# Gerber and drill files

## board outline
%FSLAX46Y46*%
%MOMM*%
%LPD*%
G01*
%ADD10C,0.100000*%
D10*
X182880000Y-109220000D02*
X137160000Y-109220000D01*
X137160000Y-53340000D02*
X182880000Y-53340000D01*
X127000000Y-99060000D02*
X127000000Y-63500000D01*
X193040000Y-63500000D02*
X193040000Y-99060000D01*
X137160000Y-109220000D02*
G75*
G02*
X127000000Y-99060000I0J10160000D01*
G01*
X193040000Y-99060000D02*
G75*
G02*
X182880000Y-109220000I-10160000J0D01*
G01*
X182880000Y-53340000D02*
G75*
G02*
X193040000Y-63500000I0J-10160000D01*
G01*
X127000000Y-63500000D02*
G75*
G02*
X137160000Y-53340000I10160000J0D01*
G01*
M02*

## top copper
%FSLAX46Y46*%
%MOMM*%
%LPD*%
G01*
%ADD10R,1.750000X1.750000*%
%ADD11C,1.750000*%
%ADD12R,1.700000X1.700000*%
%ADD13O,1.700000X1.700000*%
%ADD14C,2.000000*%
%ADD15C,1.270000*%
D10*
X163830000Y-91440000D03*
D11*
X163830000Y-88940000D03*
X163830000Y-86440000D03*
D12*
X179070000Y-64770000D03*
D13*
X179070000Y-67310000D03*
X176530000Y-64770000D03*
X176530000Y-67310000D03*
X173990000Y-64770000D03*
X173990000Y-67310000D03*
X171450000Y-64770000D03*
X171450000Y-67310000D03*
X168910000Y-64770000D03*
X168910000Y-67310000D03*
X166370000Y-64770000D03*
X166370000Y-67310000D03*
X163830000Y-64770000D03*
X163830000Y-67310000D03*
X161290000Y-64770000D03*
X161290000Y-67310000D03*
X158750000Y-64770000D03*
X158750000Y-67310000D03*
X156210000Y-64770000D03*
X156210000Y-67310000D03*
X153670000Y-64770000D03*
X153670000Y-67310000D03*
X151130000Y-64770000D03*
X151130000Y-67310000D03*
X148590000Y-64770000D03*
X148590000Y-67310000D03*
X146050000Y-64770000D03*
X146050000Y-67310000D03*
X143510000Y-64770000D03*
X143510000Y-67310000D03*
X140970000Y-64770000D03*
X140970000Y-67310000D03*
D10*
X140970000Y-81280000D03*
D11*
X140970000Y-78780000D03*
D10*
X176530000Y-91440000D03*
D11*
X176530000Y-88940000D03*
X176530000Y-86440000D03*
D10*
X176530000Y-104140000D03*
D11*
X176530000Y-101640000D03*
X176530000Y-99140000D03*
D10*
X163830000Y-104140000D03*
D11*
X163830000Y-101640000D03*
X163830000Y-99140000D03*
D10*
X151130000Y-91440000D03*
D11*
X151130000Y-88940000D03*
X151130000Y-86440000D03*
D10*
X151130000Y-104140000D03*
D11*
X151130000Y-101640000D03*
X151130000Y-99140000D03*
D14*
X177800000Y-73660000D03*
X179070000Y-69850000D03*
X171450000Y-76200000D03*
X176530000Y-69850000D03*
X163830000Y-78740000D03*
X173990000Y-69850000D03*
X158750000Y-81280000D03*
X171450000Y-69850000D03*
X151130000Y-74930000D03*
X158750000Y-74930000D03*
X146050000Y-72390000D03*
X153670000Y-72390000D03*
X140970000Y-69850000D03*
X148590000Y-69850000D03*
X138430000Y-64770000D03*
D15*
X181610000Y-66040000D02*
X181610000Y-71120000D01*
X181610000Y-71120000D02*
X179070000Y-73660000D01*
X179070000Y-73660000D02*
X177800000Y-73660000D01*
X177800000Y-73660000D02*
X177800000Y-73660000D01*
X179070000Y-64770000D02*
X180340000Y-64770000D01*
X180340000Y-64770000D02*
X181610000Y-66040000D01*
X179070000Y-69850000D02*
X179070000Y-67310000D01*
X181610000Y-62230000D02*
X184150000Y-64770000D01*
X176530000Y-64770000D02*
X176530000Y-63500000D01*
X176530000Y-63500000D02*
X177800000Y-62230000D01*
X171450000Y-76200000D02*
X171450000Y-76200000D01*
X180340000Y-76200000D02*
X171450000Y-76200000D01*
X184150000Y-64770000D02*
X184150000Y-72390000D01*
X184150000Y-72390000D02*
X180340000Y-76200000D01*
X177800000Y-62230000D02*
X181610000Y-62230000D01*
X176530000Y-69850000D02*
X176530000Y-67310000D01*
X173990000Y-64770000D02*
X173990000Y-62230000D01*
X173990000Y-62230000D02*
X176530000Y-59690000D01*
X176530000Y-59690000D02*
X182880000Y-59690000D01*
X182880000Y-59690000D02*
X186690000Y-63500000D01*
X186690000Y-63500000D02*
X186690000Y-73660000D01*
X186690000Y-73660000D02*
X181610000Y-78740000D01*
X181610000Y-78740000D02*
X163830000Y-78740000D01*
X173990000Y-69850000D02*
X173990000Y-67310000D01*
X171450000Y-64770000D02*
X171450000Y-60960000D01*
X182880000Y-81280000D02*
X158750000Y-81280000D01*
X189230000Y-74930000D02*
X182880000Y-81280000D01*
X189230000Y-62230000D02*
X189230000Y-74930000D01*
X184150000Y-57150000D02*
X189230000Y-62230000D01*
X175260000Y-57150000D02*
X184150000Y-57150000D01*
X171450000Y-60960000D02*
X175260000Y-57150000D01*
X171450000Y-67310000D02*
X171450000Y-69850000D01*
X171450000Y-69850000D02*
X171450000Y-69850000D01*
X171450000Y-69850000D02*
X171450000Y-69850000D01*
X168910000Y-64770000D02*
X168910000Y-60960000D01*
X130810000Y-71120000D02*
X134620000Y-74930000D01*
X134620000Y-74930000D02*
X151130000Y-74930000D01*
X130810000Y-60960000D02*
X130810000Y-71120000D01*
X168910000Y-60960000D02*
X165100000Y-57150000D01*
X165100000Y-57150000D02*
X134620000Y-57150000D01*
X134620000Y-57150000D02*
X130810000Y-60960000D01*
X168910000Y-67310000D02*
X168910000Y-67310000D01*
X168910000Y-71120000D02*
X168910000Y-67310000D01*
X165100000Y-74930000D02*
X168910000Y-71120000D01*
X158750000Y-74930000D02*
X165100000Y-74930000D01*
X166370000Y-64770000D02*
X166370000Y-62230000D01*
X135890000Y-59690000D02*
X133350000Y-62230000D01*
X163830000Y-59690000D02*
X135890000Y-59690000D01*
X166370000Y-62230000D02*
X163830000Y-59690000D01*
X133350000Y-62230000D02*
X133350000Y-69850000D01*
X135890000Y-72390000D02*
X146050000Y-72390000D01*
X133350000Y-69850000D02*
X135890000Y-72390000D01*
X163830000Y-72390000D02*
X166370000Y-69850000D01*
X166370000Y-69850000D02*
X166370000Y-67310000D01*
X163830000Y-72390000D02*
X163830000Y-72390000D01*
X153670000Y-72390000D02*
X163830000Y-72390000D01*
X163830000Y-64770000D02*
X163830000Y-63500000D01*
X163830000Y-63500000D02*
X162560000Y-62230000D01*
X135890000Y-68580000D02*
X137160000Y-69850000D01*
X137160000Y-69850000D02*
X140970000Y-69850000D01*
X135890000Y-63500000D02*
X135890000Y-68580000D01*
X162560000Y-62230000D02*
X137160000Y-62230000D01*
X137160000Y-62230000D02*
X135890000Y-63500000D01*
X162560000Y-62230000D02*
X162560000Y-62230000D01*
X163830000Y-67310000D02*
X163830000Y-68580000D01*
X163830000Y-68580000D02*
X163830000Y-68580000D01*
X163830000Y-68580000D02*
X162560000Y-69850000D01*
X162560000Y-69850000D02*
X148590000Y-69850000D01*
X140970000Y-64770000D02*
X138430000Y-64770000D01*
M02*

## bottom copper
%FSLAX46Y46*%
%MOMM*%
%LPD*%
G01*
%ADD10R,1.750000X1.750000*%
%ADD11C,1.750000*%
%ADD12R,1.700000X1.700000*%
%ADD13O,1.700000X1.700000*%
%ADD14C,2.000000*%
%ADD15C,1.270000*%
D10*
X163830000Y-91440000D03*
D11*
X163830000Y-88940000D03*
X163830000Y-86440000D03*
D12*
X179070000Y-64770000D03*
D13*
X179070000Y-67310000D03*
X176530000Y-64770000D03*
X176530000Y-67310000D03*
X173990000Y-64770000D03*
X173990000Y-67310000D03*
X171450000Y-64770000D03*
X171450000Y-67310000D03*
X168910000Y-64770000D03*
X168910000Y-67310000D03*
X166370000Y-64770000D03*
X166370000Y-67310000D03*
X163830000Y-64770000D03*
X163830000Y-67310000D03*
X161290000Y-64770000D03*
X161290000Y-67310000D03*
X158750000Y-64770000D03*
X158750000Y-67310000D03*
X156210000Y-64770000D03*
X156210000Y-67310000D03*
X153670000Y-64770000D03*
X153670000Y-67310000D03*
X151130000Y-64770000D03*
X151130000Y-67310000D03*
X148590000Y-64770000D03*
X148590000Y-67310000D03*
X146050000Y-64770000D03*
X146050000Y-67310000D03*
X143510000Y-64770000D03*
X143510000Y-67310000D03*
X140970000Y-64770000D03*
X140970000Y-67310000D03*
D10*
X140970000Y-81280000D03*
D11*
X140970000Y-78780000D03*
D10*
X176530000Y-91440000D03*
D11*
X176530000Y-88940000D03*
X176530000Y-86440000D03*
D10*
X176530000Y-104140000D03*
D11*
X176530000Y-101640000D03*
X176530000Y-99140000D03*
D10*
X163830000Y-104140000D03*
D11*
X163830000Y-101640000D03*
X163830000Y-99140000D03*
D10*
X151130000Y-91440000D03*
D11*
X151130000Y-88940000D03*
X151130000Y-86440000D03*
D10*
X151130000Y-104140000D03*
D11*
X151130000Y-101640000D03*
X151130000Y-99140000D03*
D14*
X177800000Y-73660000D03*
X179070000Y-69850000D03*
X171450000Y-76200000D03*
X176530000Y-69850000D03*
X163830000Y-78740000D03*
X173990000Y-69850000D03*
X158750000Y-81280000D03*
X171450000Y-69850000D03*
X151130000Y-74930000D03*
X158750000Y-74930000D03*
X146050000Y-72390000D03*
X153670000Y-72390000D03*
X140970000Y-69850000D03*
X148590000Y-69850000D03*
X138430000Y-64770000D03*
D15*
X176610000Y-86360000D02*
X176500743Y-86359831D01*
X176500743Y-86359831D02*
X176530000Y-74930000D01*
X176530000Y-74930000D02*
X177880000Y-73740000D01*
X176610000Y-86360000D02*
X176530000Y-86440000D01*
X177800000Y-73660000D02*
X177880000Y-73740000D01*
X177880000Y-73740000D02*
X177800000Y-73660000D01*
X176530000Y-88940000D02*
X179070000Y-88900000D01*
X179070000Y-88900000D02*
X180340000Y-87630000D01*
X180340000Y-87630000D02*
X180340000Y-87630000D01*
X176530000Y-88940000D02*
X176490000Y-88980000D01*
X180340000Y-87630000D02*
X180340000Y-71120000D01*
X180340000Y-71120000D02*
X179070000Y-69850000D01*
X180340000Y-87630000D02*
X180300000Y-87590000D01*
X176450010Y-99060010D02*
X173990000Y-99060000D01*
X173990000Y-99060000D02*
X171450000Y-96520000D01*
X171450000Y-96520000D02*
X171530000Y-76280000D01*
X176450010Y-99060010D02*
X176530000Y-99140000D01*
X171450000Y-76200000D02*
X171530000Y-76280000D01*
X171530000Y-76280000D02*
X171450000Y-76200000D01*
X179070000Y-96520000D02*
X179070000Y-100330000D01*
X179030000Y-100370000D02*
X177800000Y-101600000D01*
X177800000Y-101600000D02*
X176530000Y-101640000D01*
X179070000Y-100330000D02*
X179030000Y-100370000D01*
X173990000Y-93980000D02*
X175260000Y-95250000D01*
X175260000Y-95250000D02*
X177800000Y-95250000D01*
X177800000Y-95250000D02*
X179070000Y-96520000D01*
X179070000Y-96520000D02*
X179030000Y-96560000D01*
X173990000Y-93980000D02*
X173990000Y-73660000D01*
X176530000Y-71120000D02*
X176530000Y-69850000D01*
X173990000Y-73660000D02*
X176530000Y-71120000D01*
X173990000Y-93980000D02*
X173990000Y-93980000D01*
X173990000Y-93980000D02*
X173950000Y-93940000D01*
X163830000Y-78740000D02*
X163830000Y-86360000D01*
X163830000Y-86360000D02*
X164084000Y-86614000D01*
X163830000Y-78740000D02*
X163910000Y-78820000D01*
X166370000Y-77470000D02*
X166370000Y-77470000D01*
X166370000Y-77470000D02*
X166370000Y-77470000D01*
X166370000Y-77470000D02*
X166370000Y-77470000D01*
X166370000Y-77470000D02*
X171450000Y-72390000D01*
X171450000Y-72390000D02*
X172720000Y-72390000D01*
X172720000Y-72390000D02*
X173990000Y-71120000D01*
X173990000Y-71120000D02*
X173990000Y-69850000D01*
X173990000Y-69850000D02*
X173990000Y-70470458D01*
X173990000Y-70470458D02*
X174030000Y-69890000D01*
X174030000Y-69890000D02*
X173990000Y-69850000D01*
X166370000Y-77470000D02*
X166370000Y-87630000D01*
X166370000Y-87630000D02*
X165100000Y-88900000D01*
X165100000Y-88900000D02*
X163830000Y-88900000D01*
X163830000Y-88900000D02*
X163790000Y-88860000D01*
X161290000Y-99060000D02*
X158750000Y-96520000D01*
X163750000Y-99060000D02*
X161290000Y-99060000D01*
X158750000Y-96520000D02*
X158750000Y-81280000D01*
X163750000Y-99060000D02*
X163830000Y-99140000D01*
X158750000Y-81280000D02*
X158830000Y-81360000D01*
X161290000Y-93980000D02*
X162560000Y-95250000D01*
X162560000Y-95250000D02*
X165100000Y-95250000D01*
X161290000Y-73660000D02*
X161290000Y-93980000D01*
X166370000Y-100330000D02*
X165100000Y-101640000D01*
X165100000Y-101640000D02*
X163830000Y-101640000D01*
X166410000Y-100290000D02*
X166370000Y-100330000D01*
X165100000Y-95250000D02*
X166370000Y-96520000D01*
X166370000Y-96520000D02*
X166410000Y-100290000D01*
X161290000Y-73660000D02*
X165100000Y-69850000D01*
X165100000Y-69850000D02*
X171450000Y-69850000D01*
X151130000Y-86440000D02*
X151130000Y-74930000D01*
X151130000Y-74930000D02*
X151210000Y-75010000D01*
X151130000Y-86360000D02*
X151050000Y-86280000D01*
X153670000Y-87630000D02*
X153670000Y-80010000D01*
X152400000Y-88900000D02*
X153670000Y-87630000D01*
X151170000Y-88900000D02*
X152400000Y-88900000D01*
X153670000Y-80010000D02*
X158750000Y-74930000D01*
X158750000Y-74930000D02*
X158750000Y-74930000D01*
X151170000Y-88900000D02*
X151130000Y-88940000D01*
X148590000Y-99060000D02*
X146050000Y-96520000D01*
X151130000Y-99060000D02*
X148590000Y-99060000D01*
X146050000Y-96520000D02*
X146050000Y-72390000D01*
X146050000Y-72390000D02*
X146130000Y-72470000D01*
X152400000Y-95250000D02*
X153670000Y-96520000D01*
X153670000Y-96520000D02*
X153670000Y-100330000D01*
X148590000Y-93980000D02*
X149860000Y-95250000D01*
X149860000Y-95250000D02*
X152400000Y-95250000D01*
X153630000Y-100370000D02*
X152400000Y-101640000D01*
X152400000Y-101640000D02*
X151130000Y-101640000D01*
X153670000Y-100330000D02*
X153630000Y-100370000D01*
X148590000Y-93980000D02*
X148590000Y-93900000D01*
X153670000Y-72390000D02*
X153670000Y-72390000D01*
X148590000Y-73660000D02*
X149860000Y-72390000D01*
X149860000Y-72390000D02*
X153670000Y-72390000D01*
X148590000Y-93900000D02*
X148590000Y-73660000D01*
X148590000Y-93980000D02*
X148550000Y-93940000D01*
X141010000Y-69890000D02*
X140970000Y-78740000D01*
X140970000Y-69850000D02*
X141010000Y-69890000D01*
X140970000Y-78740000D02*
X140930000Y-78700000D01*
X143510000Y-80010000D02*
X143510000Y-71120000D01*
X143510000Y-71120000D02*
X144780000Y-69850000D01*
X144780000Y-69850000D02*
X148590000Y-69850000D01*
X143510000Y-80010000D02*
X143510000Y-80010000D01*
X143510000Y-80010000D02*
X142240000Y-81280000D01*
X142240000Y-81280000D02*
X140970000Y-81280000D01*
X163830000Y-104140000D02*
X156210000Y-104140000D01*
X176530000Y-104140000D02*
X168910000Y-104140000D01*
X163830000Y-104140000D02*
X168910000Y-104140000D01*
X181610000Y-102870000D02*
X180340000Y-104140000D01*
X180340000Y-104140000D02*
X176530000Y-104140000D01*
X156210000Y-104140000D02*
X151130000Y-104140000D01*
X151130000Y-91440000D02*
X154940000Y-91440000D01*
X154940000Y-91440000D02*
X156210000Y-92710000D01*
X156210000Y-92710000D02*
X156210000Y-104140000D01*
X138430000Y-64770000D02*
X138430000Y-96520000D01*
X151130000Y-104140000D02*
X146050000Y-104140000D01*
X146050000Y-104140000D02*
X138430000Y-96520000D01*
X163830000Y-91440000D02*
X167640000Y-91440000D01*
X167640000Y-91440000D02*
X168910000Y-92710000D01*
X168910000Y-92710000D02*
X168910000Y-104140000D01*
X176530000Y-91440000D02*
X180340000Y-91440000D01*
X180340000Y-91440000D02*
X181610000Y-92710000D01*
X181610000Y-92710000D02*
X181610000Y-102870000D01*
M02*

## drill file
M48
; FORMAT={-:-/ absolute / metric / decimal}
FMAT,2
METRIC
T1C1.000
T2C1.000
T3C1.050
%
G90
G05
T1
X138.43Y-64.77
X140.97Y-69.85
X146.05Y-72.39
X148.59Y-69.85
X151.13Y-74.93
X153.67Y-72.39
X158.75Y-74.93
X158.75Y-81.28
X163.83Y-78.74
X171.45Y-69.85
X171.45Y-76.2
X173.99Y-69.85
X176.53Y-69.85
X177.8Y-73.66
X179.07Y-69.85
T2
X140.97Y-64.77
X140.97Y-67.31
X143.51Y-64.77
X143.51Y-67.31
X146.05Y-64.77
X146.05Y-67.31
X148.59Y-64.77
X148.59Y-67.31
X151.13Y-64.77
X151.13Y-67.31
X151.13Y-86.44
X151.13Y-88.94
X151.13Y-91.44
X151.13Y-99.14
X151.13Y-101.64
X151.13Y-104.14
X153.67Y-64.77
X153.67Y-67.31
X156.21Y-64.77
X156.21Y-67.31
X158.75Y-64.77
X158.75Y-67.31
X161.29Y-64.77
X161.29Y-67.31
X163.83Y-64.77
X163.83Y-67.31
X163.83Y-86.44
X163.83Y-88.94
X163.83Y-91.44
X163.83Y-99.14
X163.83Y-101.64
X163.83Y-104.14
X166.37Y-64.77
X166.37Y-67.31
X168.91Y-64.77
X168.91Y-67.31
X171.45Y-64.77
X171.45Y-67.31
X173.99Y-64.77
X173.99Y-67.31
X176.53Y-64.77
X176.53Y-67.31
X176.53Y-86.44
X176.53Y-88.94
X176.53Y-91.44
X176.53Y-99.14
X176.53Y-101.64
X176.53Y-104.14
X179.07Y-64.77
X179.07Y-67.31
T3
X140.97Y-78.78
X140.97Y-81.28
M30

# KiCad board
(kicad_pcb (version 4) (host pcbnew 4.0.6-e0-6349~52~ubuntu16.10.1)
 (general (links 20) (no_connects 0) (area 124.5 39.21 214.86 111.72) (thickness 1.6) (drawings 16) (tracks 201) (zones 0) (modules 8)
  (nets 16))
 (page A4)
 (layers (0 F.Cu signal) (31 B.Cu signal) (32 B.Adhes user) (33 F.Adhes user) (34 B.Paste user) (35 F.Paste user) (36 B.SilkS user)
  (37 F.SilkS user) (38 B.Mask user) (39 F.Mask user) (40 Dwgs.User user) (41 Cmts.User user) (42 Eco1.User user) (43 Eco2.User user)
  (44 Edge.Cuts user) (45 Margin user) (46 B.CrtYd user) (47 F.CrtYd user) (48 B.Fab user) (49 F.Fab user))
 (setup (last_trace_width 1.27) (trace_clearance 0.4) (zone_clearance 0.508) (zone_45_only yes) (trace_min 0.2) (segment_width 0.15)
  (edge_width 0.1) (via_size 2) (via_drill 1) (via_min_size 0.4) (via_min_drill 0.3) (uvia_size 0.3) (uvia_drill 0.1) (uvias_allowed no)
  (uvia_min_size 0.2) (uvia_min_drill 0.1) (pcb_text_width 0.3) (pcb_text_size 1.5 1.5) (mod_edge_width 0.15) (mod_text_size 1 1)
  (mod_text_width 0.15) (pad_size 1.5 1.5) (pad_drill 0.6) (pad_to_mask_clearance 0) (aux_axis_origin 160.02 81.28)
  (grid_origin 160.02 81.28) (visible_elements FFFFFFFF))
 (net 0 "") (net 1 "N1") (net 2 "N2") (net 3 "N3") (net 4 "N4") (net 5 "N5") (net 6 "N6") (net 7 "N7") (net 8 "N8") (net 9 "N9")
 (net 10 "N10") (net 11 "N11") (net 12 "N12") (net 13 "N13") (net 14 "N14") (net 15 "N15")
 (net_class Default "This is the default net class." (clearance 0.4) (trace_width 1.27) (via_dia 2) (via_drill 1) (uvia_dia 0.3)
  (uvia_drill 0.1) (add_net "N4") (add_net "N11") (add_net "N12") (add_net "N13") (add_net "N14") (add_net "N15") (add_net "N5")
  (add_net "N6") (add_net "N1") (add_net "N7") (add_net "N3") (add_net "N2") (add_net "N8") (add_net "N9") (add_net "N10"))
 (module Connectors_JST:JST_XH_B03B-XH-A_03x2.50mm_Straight (layer F.Cu) (at 163.83 91.44 90)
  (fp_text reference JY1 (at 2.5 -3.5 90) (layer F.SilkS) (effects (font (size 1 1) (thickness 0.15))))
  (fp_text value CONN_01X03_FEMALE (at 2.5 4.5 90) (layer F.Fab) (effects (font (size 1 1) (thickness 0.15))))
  (pad 1 thru_hole rect (at 0 0 90) (size 1.75 1.75) (drill 1) (layers *.Cu *.Mask) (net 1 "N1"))
  (pad 2 thru_hole circle (at 2.5 0 90) (size 1.75 1.75) (drill 1) (layers *.Cu *.Mask) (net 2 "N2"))
  (pad 3 thru_hole circle (at 5 0 90) (size 1.75 1.75) (drill 1) (layers *.Cu *.Mask) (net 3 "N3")))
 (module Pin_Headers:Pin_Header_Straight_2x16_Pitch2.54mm (layer F.Cu) (at 179.07 64.77 270)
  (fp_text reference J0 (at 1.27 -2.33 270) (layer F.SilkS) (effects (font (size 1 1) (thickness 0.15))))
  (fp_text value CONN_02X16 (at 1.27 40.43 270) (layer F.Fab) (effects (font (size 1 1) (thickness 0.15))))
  (pad 1 thru_hole rect (at 0 0 270) (size 1.7 1.7) (drill 1) (layers *.Cu *.Mask) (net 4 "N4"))
  (pad 2 thru_hole oval (at 2.54 0 270) (size 1.7 1.7) (drill 1) (layers *.Cu *.Mask) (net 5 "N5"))
  (pad 3 thru_hole oval (at 0 2.54 270) (size 1.7 1.7) (drill 1) (layers *.Cu *.Mask) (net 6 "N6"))
  (pad 4 thru_hole oval (at 2.54 2.54 270) (size 1.7 1.7) (drill 1) (layers *.Cu *.Mask) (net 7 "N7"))
  (pad 5 thru_hole oval (at 0 5.08 270) (size 1.7 1.7) (drill 1) (layers *.Cu *.Mask) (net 3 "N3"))
  (pad 6 thru_hole oval (at 2.54 5.08 270) (size 1.7 1.7) (drill 1) (layers *.Cu *.Mask) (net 2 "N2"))
  (pad 7 thru_hole oval (at 0 7.62 270) (size 1.7 1.7) (drill 1) (layers *.Cu *.Mask) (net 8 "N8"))
  (pad 8 thru_hole oval (at 2.54 7.62 270) (size 1.7 1.7) (drill 1) (layers *.Cu *.Mask) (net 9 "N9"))
  (pad 9 thru_hole oval (at 0 10.16 270) (size 1.7 1.7) (drill 1) (layers *.Cu *.Mask) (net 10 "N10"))
  (pad 10 thru_hole oval (at 2.54 10.16 270) (size 1.7 1.7) (drill 1) (layers *.Cu *.Mask) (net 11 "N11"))
  (pad 11 thru_hole oval (at 0 12.7 270) (size 1.7 1.7) (drill 1) (layers *.Cu *.Mask) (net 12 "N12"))
  (pad 12 thru_hole oval (at 2.54 12.7 270) (size 1.7 1.7) (drill 1) (layers *.Cu *.Mask) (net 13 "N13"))
  (pad 13 thru_hole oval (at 0 15.24 270) (size 1.7 1.7) (drill 1) (layers *.Cu *.Mask) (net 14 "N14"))
  (pad 14 thru_hole oval (at 2.54 15.24 270) (size 1.7 1.7) (drill 1) (layers *.Cu *.Mask) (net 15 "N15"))
  (pad 15 thru_hole oval (at 0 17.78 270) (size 1.7 1.7) (drill 1) (layers *.Cu *.Mask))
  (pad 16 thru_hole oval (at 2.54 17.78 270) (size 1.7 1.7) (drill 1) (layers *.Cu *.Mask))
  (pad 17 thru_hole oval (at 0 20.32 270) (size 1.7 1.7) (drill 1) (layers *.Cu *.Mask))
  (pad 18 thru_hole oval (at 2.54 20.32 270) (size 1.7 1.7) (drill 1) (layers *.Cu *.Mask))
  (pad 19 thru_hole oval (at 0 22.86 270) (size 1.7 1.7) (drill 1) (layers *.Cu *.Mask))
  (pad 20 thru_hole oval (at 2.54 22.86 270) (size 1.7 1.7) (drill 1) (layers *.Cu *.Mask))
  (pad 21 thru_hole oval (at 0 25.4 270) (size 1.7 1.7) (drill 1) (layers *.Cu *.Mask))
  (pad 22 thru_hole oval (at 2.54 25.4 270) (size 1.7 1.7) (drill 1) (layers *.Cu *.Mask))
  (pad 23 thru_hole oval (at 0 27.94 270) (size 1.7 1.7) (drill 1) (layers *.Cu *.Mask))
  (pad 24 thru_hole oval (at 2.54 27.94 270) (size 1.7 1.7) (drill 1) (layers *.Cu *.Mask))
  (pad 25 thru_hole oval (at 0 30.48 270) (size 1.7 1.7) (drill 1) (layers *.Cu *.Mask))
  (pad 26 thru_hole oval (at 2.54 30.48 270) (size 1.7 1.7) (drill 1) (layers *.Cu *.Mask))
  (pad 27 thru_hole oval (at 0 33.02 270) (size 1.7 1.7) (drill 1) (layers *.Cu *.Mask))
  (pad 28 thru_hole oval (at 2.54 33.02 270) (size 1.7 1.7) (drill 1) (layers *.Cu *.Mask))
  (pad 29 thru_hole oval (at 0 35.56 270) (size 1.7 1.7) (drill 1) (layers *.Cu *.Mask))
  (pad 30 thru_hole oval (at 2.54 35.56 270) (size 1.7 1.7) (drill 1) (layers *.Cu *.Mask))
  (pad 31 thru_hole oval (at 0 38.1 270) (size 1.7 1.7) (drill 1) (layers *.Cu *.Mask) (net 1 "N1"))
  (pad 32 thru_hole oval (at 2.54 38.1 270) (size 1.7 1.7) (drill 1) (layers *.Cu *.Mask)))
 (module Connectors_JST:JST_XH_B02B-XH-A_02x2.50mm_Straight (layer F.Cu) (at 140.97 81.28 90)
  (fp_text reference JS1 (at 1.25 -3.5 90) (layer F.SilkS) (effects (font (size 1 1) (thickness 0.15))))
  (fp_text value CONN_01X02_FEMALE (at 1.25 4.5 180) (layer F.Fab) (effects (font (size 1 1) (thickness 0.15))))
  (pad 1 thru_hole rect (at 0 0 90) (size 1.75 1.75) (drill 1.05) (layers *.Cu *.Mask) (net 15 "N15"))
  (pad 2 thru_hole circle (at 2.5 0 90) (size 1.75 1.75) (drill 1.05) (layers *.Cu *.Mask) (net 14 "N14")))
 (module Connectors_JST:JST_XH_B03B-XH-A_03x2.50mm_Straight (layer F.Cu) (at 176.53 91.44 90)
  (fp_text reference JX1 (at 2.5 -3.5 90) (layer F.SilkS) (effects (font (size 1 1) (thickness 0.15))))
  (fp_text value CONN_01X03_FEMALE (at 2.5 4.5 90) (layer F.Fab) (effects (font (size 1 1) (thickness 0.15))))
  (pad 1 thru_hole rect (at 0 0 90) (size 1.75 1.75) (drill 1) (layers *.Cu *.Mask) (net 1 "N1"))
  (pad 2 thru_hole circle (at 2.5 0 90) (size 1.75 1.75) (drill 1) (layers *.Cu *.Mask) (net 5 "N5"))
  (pad 3 thru_hole circle (at 5 0 90) (size 1.75 1.75) (drill 1) (layers *.Cu *.Mask) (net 4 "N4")))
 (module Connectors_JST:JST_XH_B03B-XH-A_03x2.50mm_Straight (layer F.Cu) (at 176.53 104.14 90)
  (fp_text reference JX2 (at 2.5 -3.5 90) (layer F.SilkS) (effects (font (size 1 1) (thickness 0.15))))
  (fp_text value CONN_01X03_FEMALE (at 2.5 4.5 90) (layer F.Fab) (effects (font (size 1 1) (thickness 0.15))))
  (pad 1 thru_hole rect (at 0 0 90) (size 1.75 1.75) (drill 1) (layers *.Cu *.Mask) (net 1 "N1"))
  (pad 2 thru_hole circle (at 2.5 0 90) (size 1.75 1.75) (drill 1) (layers *.Cu *.Mask) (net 7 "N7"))
  (pad 3 thru_hole circle (at 5 0 90) (size 1.75 1.75) (drill 1) (layers *.Cu *.Mask) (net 6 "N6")))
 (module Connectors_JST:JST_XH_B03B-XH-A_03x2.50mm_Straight (layer F.Cu) (at 163.83 104.14 90)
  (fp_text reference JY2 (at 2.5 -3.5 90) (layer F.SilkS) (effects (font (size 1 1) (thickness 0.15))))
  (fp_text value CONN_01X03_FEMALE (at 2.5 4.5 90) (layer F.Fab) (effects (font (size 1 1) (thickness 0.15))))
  (pad 1 thru_hole rect (at 0 0 90) (size 1.75 1.75) (drill 1) (layers *.Cu *.Mask) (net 1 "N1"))
  (pad 2 thru_hole circle (at 2.5 0 90) (size 1.75 1.75) (drill 1) (layers *.Cu *.Mask) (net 9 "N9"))
  (pad 3 thru_hole circle (at 5 0 90) (size 1.75 1.75) (drill 1) (layers *.Cu *.Mask) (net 8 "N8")))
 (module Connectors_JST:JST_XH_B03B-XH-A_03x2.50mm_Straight (layer F.Cu) (at 151.13 91.44 90)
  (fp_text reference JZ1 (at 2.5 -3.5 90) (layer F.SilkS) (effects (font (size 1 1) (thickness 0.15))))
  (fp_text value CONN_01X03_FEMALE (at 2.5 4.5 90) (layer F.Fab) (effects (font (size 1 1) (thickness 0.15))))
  (pad 1 thru_hole rect (at 0 0 90) (size 1.75 1.75) (drill 1) (layers *.Cu *.Mask) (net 1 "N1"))
  (pad 2 thru_hole circle (at 2.5 0 90) (size 1.75 1.75) (drill 1) (layers *.Cu *.Mask) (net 11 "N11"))
  (pad 3 thru_hole circle (at 5 0 90) (size 1.75 1.75) (drill 1) (layers *.Cu *.Mask) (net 10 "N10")))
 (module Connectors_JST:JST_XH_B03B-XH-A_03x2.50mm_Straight (layer F.Cu) (at 151.13 104.14 90)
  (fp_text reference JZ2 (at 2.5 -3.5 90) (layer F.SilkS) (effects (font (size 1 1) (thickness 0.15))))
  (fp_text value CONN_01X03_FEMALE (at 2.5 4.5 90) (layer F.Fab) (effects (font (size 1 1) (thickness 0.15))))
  (pad 1 thru_hole rect (at 0 0 90) (size 1.75 1.75) (drill 1) (layers *.Cu *.Mask) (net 1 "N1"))
  (pad 2 thru_hole circle (at 2.5 0 90) (size 1.75 1.75) (drill 1) (layers *.Cu *.Mask) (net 13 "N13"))
  (pad 3 thru_hole circle (at 5 0 90) (size 1.75 1.75) (drill 1) (layers *.Cu *.Mask) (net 12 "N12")))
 (gr_line (start 182.88 109.22) (end 137.16 109.22) (angle 90) (layer Edge.Cuts) (width 0.1))
 (gr_line (start 137.16 53.34) (end 182.88 53.34) (angle 90) (layer Edge.Cuts) (width 0.1))
 (gr_line (start 127 99.06) (end 127 63.5) (angle 90) (layer Edge.Cuts) (width 0.1))
 (gr_line (start 193.04 63.5) (end 193.04 99.06) (angle 90) (layer Edge.Cuts) (width 0.1))
 (gr_arc (start 137.16 99.06) (end 137.16 109.22) (angle 90) (layer Edge.Cuts) (width 0.1))
 (gr_arc (start 182.88 99.06) (end 193.04 99.06) (angle 90) (layer Edge.Cuts) (width 0.1))
 (gr_arc (start 182.88 63.5) (end 182.88 53.34) (angle 90) (layer Edge.Cuts) (width 0.1))
 (gr_arc (start 137.16 63.5) (end 127 63.5) (angle 90) (layer Edge.Cuts) (width 0.1))
 (segment (start 176.61 86.36) (end 176.500743 86.359831) (width 1.27) (layer B.Cu) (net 4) (status 30))
 (segment (start 176.500743 86.359831) (end 176.53 74.93) (width 1.27) (layer B.Cu) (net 4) (status 10))
 (segment (start 176.53 74.93) (end 177.88 73.74) (width 1.27) (layer B.Cu) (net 4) (status 10))
 (segment (start 176.61 86.36) (end 176.53 86.44) (width 1.27) (layer B.Cu) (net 4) (status 30))
 (segment (start 181.61 66.04) (end 181.61 71.12) (width 1.27) (layer F.Cu) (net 4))
 (segment (start 181.61 71.12) (end 179.07 73.66) (width 1.27) (layer F.Cu) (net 4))
 (segment (start 179.07 73.66) (end 177.8 73.66) (width 1.27) (layer F.Cu) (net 4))
 (segment (start 177.8 73.66) (end 177.8 73.66) (width 1.27) (layer F.Cu) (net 4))
 (segment (start 179.07 64.77) (end 180.34 64.77) (width 1.27) (layer F.Cu) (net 4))
 (segment (start 180.34 64.77) (end 181.61 66.04) (width 1.27) (layer F.Cu) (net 4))
 (segment (start 177.8 73.66) (end 177.88 73.74) (width 1.27) (layer B.Cu) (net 4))
 (segment (start 177.88 73.74) (end 177.8 73.66) (width 1.27) (layer B.Cu) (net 4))
 (segment (start 176.53 88.94) (end 179.07 88.9) (width 1.27) (layer B.Cu) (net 5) (status 10))
 (segment (start 179.07 88.9) (end 180.34 87.63) (width 1.27) (layer B.Cu) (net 5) (status 10))
 (segment (start 180.34 87.63) (end 180.34 87.63) (width 1.27) (layer B.Cu) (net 5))
 (segment (start 176.53 88.94) (end 176.49 88.98) (width 1.27) (layer B.Cu) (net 5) (status 30))
 (segment (start 180.34 87.63) (end 180.34 71.12) (width 1.27) (layer B.Cu) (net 5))
 (segment (start 180.34 71.12) (end 179.07 69.85) (width 1.27) (layer B.Cu) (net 5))
 (segment (start 179.07 69.85) (end 179.07 67.31) (width 1.27) (layer F.Cu) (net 5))
 (segment (start 180.34 87.63) (end 180.3 87.59) (width 1.27) (layer B.Cu) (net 5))
 (segment (start 181.61 62.23) (end 184.15 64.77) (width 1.27) (layer F.Cu) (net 6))
 (segment (start 176.45001 99.06001) (end 173.99 99.06) (width 1.27) (layer B.Cu) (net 6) (status 10))
 (segment (start 173.99 99.06) (end 171.45 96.52) (width 1.27) (layer B.Cu) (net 6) (status 10))
 (segment (start 171.45 96.52) (end 171.53 76.28) (width 1.27) (layer B.Cu) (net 6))
 (segment (start 176.45001 99.06001) (end 176.53 99.14) (width 1.27) (layer B.Cu) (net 6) (status 30))
 (segment (start 176.53 64.77) (end 176.53 63.5) (width 1.27) (layer F.Cu) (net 6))
 (segment (start 176.53 63.5) (end 177.8 62.23) (width 1.27) (layer F.Cu) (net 6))
 (segment (start 171.45 76.2) (end 171.45 76.2) (width 1.27) (layer F.Cu) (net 6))
 (segment (start 180.34 76.2) (end 171.45 76.2) (width 1.27) (layer F.Cu) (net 6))
 (segment (start 184.15 64.77) (end 184.15 72.39) (width 1.27) (layer F.Cu) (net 6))
 (segment (start 184.15 72.39) (end 180.34 76.2) (width 1.27) (layer F.Cu) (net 6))
 (segment (start 177.8 62.23) (end 181.61 62.23) (width 1.27) (layer F.Cu) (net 6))
 (segment (start 171.45 76.2) (end 171.53 76.28) (width 1.27) (layer B.Cu) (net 6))
 (segment (start 171.53 76.28) (end 171.45 76.2) (width 1.27) (layer B.Cu) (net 6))
 (segment (start 179.07 96.52) (end 179.07 100.33) (width 1.27) (layer B.Cu) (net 7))
 (segment (start 179.03 100.37) (end 177.8 101.6) (width 1.27) (layer B.Cu) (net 7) (status 20))
 (segment (start 177.8 101.6) (end 176.53 101.64) (width 1.27) (layer B.Cu) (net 7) (status 20))
 (segment (start 179.07 100.33) (end 179.03 100.37) (width 1.27) (layer B.Cu) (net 7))
 (segment (start 173.99 93.98) (end 175.26 95.25) (width 1.27) (layer B.Cu) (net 7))
 (segment (start 175.26 95.25) (end 177.8 95.25) (width 1.27) (layer B.Cu) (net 7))
 (segment (start 177.8 95.25) (end 179.07 96.52) (width 1.27) (layer B.Cu) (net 7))
 (segment (start 179.07 96.52) (end 179.03 96.56) (width 1.27) (layer B.Cu) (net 7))
 (segment (start 173.99 93.98) (end 173.99 73.66) (width 1.27) (layer B.Cu) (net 7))
 (segment (start 176.53 69.85) (end 176.53 67.31) (width 1.27) (layer F.Cu) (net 7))
 (segment (start 176.53 71.12) (end 176.53 69.85) (width 1.27) (layer B.Cu) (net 7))
 (segment (start 173.99 73.66) (end 176.53 71.12) (width 1.27) (layer B.Cu) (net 7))
 (segment (start 173.99 93.98) (end 173.99 93.98) (width 1.27) (layer B.Cu) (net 7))
 (segment (start 173.99 93.98) (end 173.95 93.94) (width 1.27) (layer B.Cu) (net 7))
 (segment (start 163.83 78.74) (end 163.83 86.36) (width 1.27) (layer B.Cu) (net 3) (status 20))
 (segment (start 163.83 86.36) (end 164.084 86.614) (width 1.27) (layer B.Cu) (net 3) (status 30))
 (segment (start 173.99 64.77) (end 173.99 62.23) (width 1.27) (layer F.Cu) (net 3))
 (segment (start 173.99 62.23) (end 176.53 59.69) (width 1.27) (layer F.Cu) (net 3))
 (segment (start 176.53 59.69) (end 182.88 59.69) (width 1.27) (layer F.Cu) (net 3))
 (segment (start 182.88 59.69) (end 186.69 63.5) (width 1.27) (layer F.Cu) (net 3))
 (segment (start 186.69 63.5) (end 186.69 73.66) (width 1.27) (layer F.Cu) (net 3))
 (segment (start 186.69 73.66) (end 181.61 78.74) (width 1.27) (layer F.Cu) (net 3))
 (segment (start 181.61 78.74) (end 163.83 78.74) (width 1.27) (layer F.Cu) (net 3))
 (segment (start 163.83 78.74) (end 163.91 78.82) (width 1.27) (layer B.Cu) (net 3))
 (segment (start 166.37 77.47) (end 166.37 77.47) (width 1.27) (layer B.Cu) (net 2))
 (segment (start 166.37 77.47) (end 166.37 77.47) (width 1.27) (layer B.Cu) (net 2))
 (segment (start 166.37 77.47) (end 166.37 77.47) (width 1.27) (layer B.Cu) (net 2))
 (segment (start 166.37 77.47) (end 171.45 72.39) (width 1.27) (layer B.Cu) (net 2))
 (segment (start 171.45 72.39) (end 172.72 72.39) (width 1.27) (layer B.Cu) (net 2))
 (segment (start 172.72 72.39) (end 173.99 71.12) (width 1.27) (layer B.Cu) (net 2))
 (segment (start 173.99 71.12) (end 173.99 69.85) (width 1.27) (layer B.Cu) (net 2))
 (segment (start 173.99 69.85) (end 173.99 70.470458) (width 1.27) (layer B.Cu) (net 2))
 (segment (start 173.99 70.470458) (end 174.03 69.89) (width 1.27) (layer B.Cu) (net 2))
 (segment (start 173.99 69.85) (end 173.99 67.31) (width 1.27) (layer F.Cu) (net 2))
 (segment (start 174.03 69.89) (end 173.99 69.85) (width 1.27) (layer B.Cu) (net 2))
 (segment (start 166.37 77.47) (end 166.37 87.63) (width 1.27) (layer B.Cu) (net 2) (status 20))
 (segment (start 166.37 87.63) (end 165.1 88.9) (width 1.27) (layer B.Cu) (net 2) (status 20))
 (segment (start 165.1 88.9) (end 163.83 88.9) (width 1.27) (layer B.Cu) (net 2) (status 20))
 (segment (start 163.83 88.9) (end 163.79 88.86) (width 1.27) (layer B.Cu) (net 2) (status 30))
 (segment (start 161.29 99.06) (end 158.75 96.52) (width 1.27) (layer B.Cu) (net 8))
 (segment (start 163.75 99.06) (end 161.29 99.06) (width 1.27) (layer B.Cu) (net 8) (status 10))
 (segment (start 158.75 96.52) (end 158.75 81.28) (width 1.27) (layer B.Cu) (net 8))
 (segment (start 163.75 99.06) (end 163.83 99.14) (width 1.27) (layer B.Cu) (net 8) (status 30))
 (segment (start 171.45 64.77) (end 171.45 60.96) (width 1.27) (layer F.Cu) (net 8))
 (segment (start 182.88 81.28) (end 158.75 81.28) (width 1.27) (layer F.Cu) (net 8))
 (segment (start 189.23 74.93) (end 182.88 81.28) (width 1.27) (layer F.Cu) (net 8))
 (segment (start 189.23 62.23) (end 189.23 74.93) (width 1.27) (layer F.Cu) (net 8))
 (segment (start 184.15 57.15) (end 189.23 62.23) (width 1.27) (layer F.Cu) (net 8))
 (segment (start 175.26 57.15) (end 184.15 57.15) (width 1.27) (layer F.Cu) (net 8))
 (segment (start 171.45 60.96) (end 175.26 57.15) (width 1.27) (layer F.Cu) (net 8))
 (segment (start 158.75 81.28) (end 158.83 81.36) (width 1.27) (layer B.Cu) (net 8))
 (segment (start 171.45 67.31) (end 171.45 69.85) (width 1.27) (layer F.Cu) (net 9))
 (segment (start 161.29 93.98) (end 162.56 95.25) (width 1.27) (layer B.Cu) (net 9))
 (segment (start 162.56 95.25) (end 165.1 95.25) (width 1.27) (layer B.Cu) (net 9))
 (segment (start 161.29 73.66) (end 161.29 93.98) (width 1.27) (layer B.Cu) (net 9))
 (segment (start 166.37 100.33) (end 165.1 101.64) (width 1.27) (layer B.Cu) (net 9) (status 20))
 (segment (start 165.1 101.64) (end 163.83 101.64) (width 1.27) (layer B.Cu) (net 9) (status 20))
 (segment (start 166.41 100.29) (end 166.37 100.33) (width 1.27) (layer B.Cu) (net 9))
 (segment (start 165.1 95.25) (end 166.37 96.52) (width 1.27) (layer B.Cu) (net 9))
 (segment (start 166.37 96.52) (end 166.41 100.29) (width 1.27) (layer B.Cu) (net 9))
 (segment (start 171.45 69.85) (end 171.45 69.85) (width 1.27) (layer F.Cu) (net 9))
 (segment (start 171.45 69.85) (end 171.45 69.85) (width 1.27) (layer F.Cu) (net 9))
 (segment (start 161.29 73.66) (end 165.1 69.85) (width 1.27) (layer B.Cu) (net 9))
 (segment (start 165.1 69.85) (end 171.45 69.85) (width 1.27) (layer B.Cu) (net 9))
 (segment (start 151.13 86.44) (end 151.13 74.93) (width 1.27) (layer B.Cu) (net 10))
 (segment (start 168.91 64.77) (end 168.91 60.96) (width 1.27) (layer F.Cu) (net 10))
 (segment (start 151.13 74.93) (end 151.21 75.01) (width 1.27) (layer B.Cu) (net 10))
 (segment (start 130.81 71.12) (end 134.62 74.93) (width 1.27) (layer F.Cu) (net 10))
 (segment (start 134.62 74.93) (end 151.13 74.93) (width 1.27) (layer F.Cu) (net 10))
 (segment (start 130.81 60.96) (end 130.81 71.12) (width 1.27) (layer F.Cu) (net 10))
 (segment (start 168.91 60.96) (end 165.1 57.15) (width 1.27) (layer F.Cu) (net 10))
 (segment (start 165.1 57.15) (end 134.62 57.15) (width 1.27) (layer F.Cu) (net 10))
 (segment (start 134.62 57.15) (end 130.81 60.96) (width 1.27) (layer F.Cu) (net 10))
 (segment (start 151.13 86.36) (end 151.05 86.28) (width 1.27) (layer B.Cu) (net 10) (status 30))
 (segment (start 153.67 87.63) (end 153.67 80.01) (width 1.27) (layer B.Cu) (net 11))
 (segment (start 152.4 88.9) (end 153.67 87.63) (width 1.27) (layer B.Cu) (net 11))
 (segment (start 151.17 88.9) (end 152.4 88.9) (width 1.27) (layer B.Cu) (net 11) (status 10))
 (segment (start 153.67 80.01) (end 158.75 74.93) (width 1.27) (layer B.Cu) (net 11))
 (segment (start 168.91 67.31) (end 168.91 67.31) (width 1.27) (layer F.Cu) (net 11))
 (segment (start 168.91 71.12) (end 168.91 67.31) (width 1.27) (layer F.Cu) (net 11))
 (segment (start 165.1 74.93) (end 168.91 71.12) (width 1.27) (layer F.Cu) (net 11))
 (segment (start 158.75 74.93) (end 165.1 74.93) (width 1.27) (layer F.Cu) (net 11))
 (segment (start 158.75 74.93) (end 158.75 74.93) (width 1.27) (layer B.Cu) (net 11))
 (segment (start 151.17 88.9) (end 151.13 88.94) (width 1.27) (layer B.Cu) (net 11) (status 30))
 (segment (start 148.59 99.06) (end 146.05 96.52) (width 1.27) (layer B.Cu) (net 12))
 (segment (start 151.13 99.06) (end 148.59 99.06) (width 1.27) (layer B.Cu) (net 12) (status 10))
 (segment (start 146.05 96.52) (end 146.05 72.39) (width 1.27) (layer B.Cu) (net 12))
 (segment (start 166.37 64.77) (end 166.37 62.23) (width 1.27) (layer F.Cu) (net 12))
 (segment (start 135.89 59.69) (end 133.35 62.23) (width 1.27) (layer F.Cu) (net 12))
 (segment (start 163.83 59.69) (end 135.89 59.69) (width 1.27) (layer F.Cu) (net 12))
 (segment (start 166.37 62.23) (end 163.83 59.69) (width 1.27) (layer F.Cu) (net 12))
 (segment (start 133.35 62.23) (end 133.35 69.85) (width 1.27) (layer F.Cu) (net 12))
 (segment (start 135.89 72.39) (end 146.05 72.39) (width 1.27) (layer F.Cu) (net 12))
 (segment (start 133.35 69.85) (end 135.89 72.39) (width 1.27) (layer F.Cu) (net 12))
 (segment (start 146.05 72.39) (end 146.13 72.47) (width 1.27) (layer B.Cu) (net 12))
 (segment (start 163.83 72.39) (end 166.37 69.85) (width 1.27) (layer F.Cu) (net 13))
 (segment (start 166.37 69.85) (end 166.37 67.31) (width 1.27) (layer F.Cu) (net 13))
 (segment (start 163.83 72.39) (end 163.83 72.39) (width 1.27) (layer F.Cu) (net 13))
 (segment (start 153.67 72.39) (end 163.83 72.39) (width 1.27) (layer F.Cu) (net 13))
 (segment (start 152.4 95.25) (end 153.67 96.52) (width 1.27) (layer B.Cu) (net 13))
 (segment (start 153.67 96.52) (end 153.67 100.33) (width 1.27) (layer B.Cu) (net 13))
 (segment (start 148.59 93.98) (end 149.86 95.25) (width 1.27) (layer B.Cu) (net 13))
 (segment (start 149.86 95.25) (end 152.4 95.25) (width 1.27) (layer B.Cu) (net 13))
 (segment (start 153.63 100.37) (end 152.4 101.64) (width 1.27) (layer B.Cu) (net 13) (status 20))
 (segment (start 152.4 101.64) (end 151.13 101.64) (width 1.27) (layer B.Cu) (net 13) (status 20))
 (segment (start 153.67 100.33) (end 153.63 100.37) (width 1.27) (layer B.Cu) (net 13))
 (segment (start 148.59 93.98) (end 148.59 93.9) (width 1.27) (layer B.Cu) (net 13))
 (segment (start 153.67 72.39) (end 153.67 72.39) (width 1.27) (layer B.Cu) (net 13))
 (segment (start 148.59 73.66) (end 149.86 72.39) (width 1.27) (layer B.Cu) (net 13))
 (segment (start 149.86 72.39) (end 153.67 72.39) (width 1.27) (layer B.Cu) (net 13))
 (segment (start 148.59 93.9) (end 148.59 73.66) (width 1.27) (layer B.Cu) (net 13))
 (segment (start 148.59 93.98) (end 148.55 93.94) (width 1.27) (layer B.Cu) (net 13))
 (segment (start 163.83 64.77) (end 163.83 63.5) (width 1.27) (layer F.Cu) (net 14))
 (segment (start 163.83 63.5) (end 162.56 62.23) (width 1.27) (layer F.Cu) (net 14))
 (segment (start 141.01 69.89) (end 140.97 78.74) (width 1.27) (layer B.Cu) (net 14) (status 20))
 (segment (start 140.97 69.85) (end 141.01 69.89) (width 1.27) (layer B.Cu) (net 14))
 (segment (start 135.89 68.58) (end 137.16 69.85) (width 1.27) (layer F.Cu) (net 14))
 (segment (start 137.16 69.85) (end 140.97 69.85) (width 1.27) (layer F.Cu) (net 14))
 (segment (start 135.89 63.5) (end 135.89 68.58) (width 1.27) (layer F.Cu) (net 14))
 (segment (start 162.56 62.23) (end 137.16 62.23) (width 1.27) (layer F.Cu) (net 14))
 (segment (start 137.16 62.23) (end 135.89 63.5) (width 1.27) (layer F.Cu) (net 14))
 (segment (start 162.56 62.23) (end 162.56 62.23) (width 1.27) (layer F.Cu) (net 14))
 (segment (start 140.97 78.74) (end 140.93 78.7) (width 1.27) (layer B.Cu) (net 14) (status 30))
 (segment (start 163.83 67.31) (end 163.83 68.58) (width 1.27) (layer F.Cu) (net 15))
 (segment (start 163.83 68.58) (end 163.83 68.58) (width 1.27) (layer F.Cu) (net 15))
 (segment (start 163.83 68.58) (end 162.56 69.85) (width 1.27) (layer F.Cu) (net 15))
 (segment (start 162.56 69.85) (end 148.59 69.85) (width 1.27) (layer F.Cu) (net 15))
 (segment (start 143.51 80.01) (end 143.51 71.12) (width 1.27) (layer B.Cu) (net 15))
 (segment (start 143.51 71.12) (end 144.78 69.85) (width 1.27) (layer B.Cu) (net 15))
 (segment (start 144.78 69.85) (end 148.59 69.85) (width 1.27) (layer B.Cu) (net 15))
 (segment (start 143.51 80.01) (end 143.51 80.01) (width 1.27) (layer B.Cu) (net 15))
 (segment (start 143.51 80.01) (end 142.24 81.28) (width 1.27) (layer B.Cu) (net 15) (status 20))
 (segment (start 142.24 81.28) (end 140.97 81.28) (width 1.27) (layer B.Cu) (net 15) (status 20))
 (segment (start 163.83 104.14) (end 156.21 104.14) (width 1.27) (layer B.Cu) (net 1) (status 10))
 (segment (start 176.53 104.14) (end 168.91 104.14) (width 1.27) (layer B.Cu) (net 1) (status 10))
 (segment (start 163.83 104.14) (end 168.91 104.14) (width 1.27) (layer B.Cu) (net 1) (status 10))
 (segment (start 181.61 102.87) (end 180.34 104.14) (width 1.27) (layer B.Cu) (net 1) (status 20))
 (segment (start 180.34 104.14) (end 176.53 104.14) (width 1.27) (layer B.Cu) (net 1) (status 20))
 (segment (start 156.21 104.14) (end 151.13 104.14) (width 1.27) (layer B.Cu) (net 1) (status 20))
 (segment (start 151.13 91.44) (end 154.94 91.44) (width 1.27) (layer B.Cu) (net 1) (status 10))
 (segment (start 154.94 91.44) (end 156.21 92.71) (width 1.27) (layer B.Cu) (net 1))
 (segment (start 156.21 92.71) (end 156.21 104.14) (width 1.27) (layer B.Cu) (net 1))
 (segment (start 138.43 64.77) (end 138.43 96.52) (width 1.27) (layer B.Cu) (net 1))
 (segment (start 140.97 64.77) (end 138.43 64.77) (width 1.27) (layer F.Cu) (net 1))
 (segment (start 151.13 104.14) (end 146.05 104.14) (width 1.27) (layer B.Cu) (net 1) (status 10))
 (segment (start 146.05 104.14) (end 138.43 96.52) (width 1.27) (layer B.Cu) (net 1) (status 10))
 (segment (start 163.83 91.44) (end 167.64 91.44) (width 1.27) (layer B.Cu) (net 1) (status 10))
 (segment (start 167.64 91.44) (end 168.91 92.71) (width 1.27) (layer B.Cu) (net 1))
 (segment (start 168.91 92.71) (end 168.91 104.14) (width 1.27) (layer B.Cu) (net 1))
 (segment (start 176.53 91.44) (end 180.34 91.44) (width 1.27) (layer B.Cu) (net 1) (status 10))
 (segment (start 180.34 91.44) (end 181.61 92.71) (width 1.27) (layer B.Cu) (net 1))
 (segment (start 181.61 92.71) (end 181.61 102.87) (width 1.27) (layer B.Cu) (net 1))
 (via (at 177.8 73.66) (size 2) (drill 1) (layers F.Cu B.Cu) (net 4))
 (via (at 179.07 69.85) (size 2) (drill 1) (layers F.Cu B.Cu) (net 5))
 (via (at 171.45 76.2) (size 2) (drill 1) (layers F.Cu B.Cu) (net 6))
 (via (at 176.53 69.85) (size 2) (drill 1) (layers F.Cu B.Cu) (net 7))
 (via (at 163.83 78.74) (size 2) (drill 1) (layers F.Cu B.Cu) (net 3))
 (via (at 173.99 69.85) (size 2) (drill 1) (layers F.Cu B.Cu) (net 2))
 (via (at 158.75 81.28) (size 2) (drill 1) (layers F.Cu B.Cu) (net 8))
 (via (at 171.45 69.85) (size 2) (drill 1) (layers F.Cu B.Cu) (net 9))
 (via (at 151.13 74.93) (size 2) (drill 1) (layers F.Cu B.Cu) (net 10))
 (via (at 158.75 74.93) (size 2) (drill 1) (layers F.Cu B.Cu) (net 11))
 (via (at 146.05 72.39) (size 2) (drill 1) (layers F.Cu B.Cu) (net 12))
 (via (at 153.67 72.39) (size 2) (drill 1) (layers F.Cu B.Cu) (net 13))
 (via (at 140.97 69.85) (size 2) (drill 1) (layers F.Cu B.Cu) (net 14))
 (via (at 148.59 69.85) (size 2) (drill 1) (layers F.Cu B.Cu) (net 15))
 (via (at 138.43 64.77) (size 2) (drill 1) (layers F.Cu B.Cu) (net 1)))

